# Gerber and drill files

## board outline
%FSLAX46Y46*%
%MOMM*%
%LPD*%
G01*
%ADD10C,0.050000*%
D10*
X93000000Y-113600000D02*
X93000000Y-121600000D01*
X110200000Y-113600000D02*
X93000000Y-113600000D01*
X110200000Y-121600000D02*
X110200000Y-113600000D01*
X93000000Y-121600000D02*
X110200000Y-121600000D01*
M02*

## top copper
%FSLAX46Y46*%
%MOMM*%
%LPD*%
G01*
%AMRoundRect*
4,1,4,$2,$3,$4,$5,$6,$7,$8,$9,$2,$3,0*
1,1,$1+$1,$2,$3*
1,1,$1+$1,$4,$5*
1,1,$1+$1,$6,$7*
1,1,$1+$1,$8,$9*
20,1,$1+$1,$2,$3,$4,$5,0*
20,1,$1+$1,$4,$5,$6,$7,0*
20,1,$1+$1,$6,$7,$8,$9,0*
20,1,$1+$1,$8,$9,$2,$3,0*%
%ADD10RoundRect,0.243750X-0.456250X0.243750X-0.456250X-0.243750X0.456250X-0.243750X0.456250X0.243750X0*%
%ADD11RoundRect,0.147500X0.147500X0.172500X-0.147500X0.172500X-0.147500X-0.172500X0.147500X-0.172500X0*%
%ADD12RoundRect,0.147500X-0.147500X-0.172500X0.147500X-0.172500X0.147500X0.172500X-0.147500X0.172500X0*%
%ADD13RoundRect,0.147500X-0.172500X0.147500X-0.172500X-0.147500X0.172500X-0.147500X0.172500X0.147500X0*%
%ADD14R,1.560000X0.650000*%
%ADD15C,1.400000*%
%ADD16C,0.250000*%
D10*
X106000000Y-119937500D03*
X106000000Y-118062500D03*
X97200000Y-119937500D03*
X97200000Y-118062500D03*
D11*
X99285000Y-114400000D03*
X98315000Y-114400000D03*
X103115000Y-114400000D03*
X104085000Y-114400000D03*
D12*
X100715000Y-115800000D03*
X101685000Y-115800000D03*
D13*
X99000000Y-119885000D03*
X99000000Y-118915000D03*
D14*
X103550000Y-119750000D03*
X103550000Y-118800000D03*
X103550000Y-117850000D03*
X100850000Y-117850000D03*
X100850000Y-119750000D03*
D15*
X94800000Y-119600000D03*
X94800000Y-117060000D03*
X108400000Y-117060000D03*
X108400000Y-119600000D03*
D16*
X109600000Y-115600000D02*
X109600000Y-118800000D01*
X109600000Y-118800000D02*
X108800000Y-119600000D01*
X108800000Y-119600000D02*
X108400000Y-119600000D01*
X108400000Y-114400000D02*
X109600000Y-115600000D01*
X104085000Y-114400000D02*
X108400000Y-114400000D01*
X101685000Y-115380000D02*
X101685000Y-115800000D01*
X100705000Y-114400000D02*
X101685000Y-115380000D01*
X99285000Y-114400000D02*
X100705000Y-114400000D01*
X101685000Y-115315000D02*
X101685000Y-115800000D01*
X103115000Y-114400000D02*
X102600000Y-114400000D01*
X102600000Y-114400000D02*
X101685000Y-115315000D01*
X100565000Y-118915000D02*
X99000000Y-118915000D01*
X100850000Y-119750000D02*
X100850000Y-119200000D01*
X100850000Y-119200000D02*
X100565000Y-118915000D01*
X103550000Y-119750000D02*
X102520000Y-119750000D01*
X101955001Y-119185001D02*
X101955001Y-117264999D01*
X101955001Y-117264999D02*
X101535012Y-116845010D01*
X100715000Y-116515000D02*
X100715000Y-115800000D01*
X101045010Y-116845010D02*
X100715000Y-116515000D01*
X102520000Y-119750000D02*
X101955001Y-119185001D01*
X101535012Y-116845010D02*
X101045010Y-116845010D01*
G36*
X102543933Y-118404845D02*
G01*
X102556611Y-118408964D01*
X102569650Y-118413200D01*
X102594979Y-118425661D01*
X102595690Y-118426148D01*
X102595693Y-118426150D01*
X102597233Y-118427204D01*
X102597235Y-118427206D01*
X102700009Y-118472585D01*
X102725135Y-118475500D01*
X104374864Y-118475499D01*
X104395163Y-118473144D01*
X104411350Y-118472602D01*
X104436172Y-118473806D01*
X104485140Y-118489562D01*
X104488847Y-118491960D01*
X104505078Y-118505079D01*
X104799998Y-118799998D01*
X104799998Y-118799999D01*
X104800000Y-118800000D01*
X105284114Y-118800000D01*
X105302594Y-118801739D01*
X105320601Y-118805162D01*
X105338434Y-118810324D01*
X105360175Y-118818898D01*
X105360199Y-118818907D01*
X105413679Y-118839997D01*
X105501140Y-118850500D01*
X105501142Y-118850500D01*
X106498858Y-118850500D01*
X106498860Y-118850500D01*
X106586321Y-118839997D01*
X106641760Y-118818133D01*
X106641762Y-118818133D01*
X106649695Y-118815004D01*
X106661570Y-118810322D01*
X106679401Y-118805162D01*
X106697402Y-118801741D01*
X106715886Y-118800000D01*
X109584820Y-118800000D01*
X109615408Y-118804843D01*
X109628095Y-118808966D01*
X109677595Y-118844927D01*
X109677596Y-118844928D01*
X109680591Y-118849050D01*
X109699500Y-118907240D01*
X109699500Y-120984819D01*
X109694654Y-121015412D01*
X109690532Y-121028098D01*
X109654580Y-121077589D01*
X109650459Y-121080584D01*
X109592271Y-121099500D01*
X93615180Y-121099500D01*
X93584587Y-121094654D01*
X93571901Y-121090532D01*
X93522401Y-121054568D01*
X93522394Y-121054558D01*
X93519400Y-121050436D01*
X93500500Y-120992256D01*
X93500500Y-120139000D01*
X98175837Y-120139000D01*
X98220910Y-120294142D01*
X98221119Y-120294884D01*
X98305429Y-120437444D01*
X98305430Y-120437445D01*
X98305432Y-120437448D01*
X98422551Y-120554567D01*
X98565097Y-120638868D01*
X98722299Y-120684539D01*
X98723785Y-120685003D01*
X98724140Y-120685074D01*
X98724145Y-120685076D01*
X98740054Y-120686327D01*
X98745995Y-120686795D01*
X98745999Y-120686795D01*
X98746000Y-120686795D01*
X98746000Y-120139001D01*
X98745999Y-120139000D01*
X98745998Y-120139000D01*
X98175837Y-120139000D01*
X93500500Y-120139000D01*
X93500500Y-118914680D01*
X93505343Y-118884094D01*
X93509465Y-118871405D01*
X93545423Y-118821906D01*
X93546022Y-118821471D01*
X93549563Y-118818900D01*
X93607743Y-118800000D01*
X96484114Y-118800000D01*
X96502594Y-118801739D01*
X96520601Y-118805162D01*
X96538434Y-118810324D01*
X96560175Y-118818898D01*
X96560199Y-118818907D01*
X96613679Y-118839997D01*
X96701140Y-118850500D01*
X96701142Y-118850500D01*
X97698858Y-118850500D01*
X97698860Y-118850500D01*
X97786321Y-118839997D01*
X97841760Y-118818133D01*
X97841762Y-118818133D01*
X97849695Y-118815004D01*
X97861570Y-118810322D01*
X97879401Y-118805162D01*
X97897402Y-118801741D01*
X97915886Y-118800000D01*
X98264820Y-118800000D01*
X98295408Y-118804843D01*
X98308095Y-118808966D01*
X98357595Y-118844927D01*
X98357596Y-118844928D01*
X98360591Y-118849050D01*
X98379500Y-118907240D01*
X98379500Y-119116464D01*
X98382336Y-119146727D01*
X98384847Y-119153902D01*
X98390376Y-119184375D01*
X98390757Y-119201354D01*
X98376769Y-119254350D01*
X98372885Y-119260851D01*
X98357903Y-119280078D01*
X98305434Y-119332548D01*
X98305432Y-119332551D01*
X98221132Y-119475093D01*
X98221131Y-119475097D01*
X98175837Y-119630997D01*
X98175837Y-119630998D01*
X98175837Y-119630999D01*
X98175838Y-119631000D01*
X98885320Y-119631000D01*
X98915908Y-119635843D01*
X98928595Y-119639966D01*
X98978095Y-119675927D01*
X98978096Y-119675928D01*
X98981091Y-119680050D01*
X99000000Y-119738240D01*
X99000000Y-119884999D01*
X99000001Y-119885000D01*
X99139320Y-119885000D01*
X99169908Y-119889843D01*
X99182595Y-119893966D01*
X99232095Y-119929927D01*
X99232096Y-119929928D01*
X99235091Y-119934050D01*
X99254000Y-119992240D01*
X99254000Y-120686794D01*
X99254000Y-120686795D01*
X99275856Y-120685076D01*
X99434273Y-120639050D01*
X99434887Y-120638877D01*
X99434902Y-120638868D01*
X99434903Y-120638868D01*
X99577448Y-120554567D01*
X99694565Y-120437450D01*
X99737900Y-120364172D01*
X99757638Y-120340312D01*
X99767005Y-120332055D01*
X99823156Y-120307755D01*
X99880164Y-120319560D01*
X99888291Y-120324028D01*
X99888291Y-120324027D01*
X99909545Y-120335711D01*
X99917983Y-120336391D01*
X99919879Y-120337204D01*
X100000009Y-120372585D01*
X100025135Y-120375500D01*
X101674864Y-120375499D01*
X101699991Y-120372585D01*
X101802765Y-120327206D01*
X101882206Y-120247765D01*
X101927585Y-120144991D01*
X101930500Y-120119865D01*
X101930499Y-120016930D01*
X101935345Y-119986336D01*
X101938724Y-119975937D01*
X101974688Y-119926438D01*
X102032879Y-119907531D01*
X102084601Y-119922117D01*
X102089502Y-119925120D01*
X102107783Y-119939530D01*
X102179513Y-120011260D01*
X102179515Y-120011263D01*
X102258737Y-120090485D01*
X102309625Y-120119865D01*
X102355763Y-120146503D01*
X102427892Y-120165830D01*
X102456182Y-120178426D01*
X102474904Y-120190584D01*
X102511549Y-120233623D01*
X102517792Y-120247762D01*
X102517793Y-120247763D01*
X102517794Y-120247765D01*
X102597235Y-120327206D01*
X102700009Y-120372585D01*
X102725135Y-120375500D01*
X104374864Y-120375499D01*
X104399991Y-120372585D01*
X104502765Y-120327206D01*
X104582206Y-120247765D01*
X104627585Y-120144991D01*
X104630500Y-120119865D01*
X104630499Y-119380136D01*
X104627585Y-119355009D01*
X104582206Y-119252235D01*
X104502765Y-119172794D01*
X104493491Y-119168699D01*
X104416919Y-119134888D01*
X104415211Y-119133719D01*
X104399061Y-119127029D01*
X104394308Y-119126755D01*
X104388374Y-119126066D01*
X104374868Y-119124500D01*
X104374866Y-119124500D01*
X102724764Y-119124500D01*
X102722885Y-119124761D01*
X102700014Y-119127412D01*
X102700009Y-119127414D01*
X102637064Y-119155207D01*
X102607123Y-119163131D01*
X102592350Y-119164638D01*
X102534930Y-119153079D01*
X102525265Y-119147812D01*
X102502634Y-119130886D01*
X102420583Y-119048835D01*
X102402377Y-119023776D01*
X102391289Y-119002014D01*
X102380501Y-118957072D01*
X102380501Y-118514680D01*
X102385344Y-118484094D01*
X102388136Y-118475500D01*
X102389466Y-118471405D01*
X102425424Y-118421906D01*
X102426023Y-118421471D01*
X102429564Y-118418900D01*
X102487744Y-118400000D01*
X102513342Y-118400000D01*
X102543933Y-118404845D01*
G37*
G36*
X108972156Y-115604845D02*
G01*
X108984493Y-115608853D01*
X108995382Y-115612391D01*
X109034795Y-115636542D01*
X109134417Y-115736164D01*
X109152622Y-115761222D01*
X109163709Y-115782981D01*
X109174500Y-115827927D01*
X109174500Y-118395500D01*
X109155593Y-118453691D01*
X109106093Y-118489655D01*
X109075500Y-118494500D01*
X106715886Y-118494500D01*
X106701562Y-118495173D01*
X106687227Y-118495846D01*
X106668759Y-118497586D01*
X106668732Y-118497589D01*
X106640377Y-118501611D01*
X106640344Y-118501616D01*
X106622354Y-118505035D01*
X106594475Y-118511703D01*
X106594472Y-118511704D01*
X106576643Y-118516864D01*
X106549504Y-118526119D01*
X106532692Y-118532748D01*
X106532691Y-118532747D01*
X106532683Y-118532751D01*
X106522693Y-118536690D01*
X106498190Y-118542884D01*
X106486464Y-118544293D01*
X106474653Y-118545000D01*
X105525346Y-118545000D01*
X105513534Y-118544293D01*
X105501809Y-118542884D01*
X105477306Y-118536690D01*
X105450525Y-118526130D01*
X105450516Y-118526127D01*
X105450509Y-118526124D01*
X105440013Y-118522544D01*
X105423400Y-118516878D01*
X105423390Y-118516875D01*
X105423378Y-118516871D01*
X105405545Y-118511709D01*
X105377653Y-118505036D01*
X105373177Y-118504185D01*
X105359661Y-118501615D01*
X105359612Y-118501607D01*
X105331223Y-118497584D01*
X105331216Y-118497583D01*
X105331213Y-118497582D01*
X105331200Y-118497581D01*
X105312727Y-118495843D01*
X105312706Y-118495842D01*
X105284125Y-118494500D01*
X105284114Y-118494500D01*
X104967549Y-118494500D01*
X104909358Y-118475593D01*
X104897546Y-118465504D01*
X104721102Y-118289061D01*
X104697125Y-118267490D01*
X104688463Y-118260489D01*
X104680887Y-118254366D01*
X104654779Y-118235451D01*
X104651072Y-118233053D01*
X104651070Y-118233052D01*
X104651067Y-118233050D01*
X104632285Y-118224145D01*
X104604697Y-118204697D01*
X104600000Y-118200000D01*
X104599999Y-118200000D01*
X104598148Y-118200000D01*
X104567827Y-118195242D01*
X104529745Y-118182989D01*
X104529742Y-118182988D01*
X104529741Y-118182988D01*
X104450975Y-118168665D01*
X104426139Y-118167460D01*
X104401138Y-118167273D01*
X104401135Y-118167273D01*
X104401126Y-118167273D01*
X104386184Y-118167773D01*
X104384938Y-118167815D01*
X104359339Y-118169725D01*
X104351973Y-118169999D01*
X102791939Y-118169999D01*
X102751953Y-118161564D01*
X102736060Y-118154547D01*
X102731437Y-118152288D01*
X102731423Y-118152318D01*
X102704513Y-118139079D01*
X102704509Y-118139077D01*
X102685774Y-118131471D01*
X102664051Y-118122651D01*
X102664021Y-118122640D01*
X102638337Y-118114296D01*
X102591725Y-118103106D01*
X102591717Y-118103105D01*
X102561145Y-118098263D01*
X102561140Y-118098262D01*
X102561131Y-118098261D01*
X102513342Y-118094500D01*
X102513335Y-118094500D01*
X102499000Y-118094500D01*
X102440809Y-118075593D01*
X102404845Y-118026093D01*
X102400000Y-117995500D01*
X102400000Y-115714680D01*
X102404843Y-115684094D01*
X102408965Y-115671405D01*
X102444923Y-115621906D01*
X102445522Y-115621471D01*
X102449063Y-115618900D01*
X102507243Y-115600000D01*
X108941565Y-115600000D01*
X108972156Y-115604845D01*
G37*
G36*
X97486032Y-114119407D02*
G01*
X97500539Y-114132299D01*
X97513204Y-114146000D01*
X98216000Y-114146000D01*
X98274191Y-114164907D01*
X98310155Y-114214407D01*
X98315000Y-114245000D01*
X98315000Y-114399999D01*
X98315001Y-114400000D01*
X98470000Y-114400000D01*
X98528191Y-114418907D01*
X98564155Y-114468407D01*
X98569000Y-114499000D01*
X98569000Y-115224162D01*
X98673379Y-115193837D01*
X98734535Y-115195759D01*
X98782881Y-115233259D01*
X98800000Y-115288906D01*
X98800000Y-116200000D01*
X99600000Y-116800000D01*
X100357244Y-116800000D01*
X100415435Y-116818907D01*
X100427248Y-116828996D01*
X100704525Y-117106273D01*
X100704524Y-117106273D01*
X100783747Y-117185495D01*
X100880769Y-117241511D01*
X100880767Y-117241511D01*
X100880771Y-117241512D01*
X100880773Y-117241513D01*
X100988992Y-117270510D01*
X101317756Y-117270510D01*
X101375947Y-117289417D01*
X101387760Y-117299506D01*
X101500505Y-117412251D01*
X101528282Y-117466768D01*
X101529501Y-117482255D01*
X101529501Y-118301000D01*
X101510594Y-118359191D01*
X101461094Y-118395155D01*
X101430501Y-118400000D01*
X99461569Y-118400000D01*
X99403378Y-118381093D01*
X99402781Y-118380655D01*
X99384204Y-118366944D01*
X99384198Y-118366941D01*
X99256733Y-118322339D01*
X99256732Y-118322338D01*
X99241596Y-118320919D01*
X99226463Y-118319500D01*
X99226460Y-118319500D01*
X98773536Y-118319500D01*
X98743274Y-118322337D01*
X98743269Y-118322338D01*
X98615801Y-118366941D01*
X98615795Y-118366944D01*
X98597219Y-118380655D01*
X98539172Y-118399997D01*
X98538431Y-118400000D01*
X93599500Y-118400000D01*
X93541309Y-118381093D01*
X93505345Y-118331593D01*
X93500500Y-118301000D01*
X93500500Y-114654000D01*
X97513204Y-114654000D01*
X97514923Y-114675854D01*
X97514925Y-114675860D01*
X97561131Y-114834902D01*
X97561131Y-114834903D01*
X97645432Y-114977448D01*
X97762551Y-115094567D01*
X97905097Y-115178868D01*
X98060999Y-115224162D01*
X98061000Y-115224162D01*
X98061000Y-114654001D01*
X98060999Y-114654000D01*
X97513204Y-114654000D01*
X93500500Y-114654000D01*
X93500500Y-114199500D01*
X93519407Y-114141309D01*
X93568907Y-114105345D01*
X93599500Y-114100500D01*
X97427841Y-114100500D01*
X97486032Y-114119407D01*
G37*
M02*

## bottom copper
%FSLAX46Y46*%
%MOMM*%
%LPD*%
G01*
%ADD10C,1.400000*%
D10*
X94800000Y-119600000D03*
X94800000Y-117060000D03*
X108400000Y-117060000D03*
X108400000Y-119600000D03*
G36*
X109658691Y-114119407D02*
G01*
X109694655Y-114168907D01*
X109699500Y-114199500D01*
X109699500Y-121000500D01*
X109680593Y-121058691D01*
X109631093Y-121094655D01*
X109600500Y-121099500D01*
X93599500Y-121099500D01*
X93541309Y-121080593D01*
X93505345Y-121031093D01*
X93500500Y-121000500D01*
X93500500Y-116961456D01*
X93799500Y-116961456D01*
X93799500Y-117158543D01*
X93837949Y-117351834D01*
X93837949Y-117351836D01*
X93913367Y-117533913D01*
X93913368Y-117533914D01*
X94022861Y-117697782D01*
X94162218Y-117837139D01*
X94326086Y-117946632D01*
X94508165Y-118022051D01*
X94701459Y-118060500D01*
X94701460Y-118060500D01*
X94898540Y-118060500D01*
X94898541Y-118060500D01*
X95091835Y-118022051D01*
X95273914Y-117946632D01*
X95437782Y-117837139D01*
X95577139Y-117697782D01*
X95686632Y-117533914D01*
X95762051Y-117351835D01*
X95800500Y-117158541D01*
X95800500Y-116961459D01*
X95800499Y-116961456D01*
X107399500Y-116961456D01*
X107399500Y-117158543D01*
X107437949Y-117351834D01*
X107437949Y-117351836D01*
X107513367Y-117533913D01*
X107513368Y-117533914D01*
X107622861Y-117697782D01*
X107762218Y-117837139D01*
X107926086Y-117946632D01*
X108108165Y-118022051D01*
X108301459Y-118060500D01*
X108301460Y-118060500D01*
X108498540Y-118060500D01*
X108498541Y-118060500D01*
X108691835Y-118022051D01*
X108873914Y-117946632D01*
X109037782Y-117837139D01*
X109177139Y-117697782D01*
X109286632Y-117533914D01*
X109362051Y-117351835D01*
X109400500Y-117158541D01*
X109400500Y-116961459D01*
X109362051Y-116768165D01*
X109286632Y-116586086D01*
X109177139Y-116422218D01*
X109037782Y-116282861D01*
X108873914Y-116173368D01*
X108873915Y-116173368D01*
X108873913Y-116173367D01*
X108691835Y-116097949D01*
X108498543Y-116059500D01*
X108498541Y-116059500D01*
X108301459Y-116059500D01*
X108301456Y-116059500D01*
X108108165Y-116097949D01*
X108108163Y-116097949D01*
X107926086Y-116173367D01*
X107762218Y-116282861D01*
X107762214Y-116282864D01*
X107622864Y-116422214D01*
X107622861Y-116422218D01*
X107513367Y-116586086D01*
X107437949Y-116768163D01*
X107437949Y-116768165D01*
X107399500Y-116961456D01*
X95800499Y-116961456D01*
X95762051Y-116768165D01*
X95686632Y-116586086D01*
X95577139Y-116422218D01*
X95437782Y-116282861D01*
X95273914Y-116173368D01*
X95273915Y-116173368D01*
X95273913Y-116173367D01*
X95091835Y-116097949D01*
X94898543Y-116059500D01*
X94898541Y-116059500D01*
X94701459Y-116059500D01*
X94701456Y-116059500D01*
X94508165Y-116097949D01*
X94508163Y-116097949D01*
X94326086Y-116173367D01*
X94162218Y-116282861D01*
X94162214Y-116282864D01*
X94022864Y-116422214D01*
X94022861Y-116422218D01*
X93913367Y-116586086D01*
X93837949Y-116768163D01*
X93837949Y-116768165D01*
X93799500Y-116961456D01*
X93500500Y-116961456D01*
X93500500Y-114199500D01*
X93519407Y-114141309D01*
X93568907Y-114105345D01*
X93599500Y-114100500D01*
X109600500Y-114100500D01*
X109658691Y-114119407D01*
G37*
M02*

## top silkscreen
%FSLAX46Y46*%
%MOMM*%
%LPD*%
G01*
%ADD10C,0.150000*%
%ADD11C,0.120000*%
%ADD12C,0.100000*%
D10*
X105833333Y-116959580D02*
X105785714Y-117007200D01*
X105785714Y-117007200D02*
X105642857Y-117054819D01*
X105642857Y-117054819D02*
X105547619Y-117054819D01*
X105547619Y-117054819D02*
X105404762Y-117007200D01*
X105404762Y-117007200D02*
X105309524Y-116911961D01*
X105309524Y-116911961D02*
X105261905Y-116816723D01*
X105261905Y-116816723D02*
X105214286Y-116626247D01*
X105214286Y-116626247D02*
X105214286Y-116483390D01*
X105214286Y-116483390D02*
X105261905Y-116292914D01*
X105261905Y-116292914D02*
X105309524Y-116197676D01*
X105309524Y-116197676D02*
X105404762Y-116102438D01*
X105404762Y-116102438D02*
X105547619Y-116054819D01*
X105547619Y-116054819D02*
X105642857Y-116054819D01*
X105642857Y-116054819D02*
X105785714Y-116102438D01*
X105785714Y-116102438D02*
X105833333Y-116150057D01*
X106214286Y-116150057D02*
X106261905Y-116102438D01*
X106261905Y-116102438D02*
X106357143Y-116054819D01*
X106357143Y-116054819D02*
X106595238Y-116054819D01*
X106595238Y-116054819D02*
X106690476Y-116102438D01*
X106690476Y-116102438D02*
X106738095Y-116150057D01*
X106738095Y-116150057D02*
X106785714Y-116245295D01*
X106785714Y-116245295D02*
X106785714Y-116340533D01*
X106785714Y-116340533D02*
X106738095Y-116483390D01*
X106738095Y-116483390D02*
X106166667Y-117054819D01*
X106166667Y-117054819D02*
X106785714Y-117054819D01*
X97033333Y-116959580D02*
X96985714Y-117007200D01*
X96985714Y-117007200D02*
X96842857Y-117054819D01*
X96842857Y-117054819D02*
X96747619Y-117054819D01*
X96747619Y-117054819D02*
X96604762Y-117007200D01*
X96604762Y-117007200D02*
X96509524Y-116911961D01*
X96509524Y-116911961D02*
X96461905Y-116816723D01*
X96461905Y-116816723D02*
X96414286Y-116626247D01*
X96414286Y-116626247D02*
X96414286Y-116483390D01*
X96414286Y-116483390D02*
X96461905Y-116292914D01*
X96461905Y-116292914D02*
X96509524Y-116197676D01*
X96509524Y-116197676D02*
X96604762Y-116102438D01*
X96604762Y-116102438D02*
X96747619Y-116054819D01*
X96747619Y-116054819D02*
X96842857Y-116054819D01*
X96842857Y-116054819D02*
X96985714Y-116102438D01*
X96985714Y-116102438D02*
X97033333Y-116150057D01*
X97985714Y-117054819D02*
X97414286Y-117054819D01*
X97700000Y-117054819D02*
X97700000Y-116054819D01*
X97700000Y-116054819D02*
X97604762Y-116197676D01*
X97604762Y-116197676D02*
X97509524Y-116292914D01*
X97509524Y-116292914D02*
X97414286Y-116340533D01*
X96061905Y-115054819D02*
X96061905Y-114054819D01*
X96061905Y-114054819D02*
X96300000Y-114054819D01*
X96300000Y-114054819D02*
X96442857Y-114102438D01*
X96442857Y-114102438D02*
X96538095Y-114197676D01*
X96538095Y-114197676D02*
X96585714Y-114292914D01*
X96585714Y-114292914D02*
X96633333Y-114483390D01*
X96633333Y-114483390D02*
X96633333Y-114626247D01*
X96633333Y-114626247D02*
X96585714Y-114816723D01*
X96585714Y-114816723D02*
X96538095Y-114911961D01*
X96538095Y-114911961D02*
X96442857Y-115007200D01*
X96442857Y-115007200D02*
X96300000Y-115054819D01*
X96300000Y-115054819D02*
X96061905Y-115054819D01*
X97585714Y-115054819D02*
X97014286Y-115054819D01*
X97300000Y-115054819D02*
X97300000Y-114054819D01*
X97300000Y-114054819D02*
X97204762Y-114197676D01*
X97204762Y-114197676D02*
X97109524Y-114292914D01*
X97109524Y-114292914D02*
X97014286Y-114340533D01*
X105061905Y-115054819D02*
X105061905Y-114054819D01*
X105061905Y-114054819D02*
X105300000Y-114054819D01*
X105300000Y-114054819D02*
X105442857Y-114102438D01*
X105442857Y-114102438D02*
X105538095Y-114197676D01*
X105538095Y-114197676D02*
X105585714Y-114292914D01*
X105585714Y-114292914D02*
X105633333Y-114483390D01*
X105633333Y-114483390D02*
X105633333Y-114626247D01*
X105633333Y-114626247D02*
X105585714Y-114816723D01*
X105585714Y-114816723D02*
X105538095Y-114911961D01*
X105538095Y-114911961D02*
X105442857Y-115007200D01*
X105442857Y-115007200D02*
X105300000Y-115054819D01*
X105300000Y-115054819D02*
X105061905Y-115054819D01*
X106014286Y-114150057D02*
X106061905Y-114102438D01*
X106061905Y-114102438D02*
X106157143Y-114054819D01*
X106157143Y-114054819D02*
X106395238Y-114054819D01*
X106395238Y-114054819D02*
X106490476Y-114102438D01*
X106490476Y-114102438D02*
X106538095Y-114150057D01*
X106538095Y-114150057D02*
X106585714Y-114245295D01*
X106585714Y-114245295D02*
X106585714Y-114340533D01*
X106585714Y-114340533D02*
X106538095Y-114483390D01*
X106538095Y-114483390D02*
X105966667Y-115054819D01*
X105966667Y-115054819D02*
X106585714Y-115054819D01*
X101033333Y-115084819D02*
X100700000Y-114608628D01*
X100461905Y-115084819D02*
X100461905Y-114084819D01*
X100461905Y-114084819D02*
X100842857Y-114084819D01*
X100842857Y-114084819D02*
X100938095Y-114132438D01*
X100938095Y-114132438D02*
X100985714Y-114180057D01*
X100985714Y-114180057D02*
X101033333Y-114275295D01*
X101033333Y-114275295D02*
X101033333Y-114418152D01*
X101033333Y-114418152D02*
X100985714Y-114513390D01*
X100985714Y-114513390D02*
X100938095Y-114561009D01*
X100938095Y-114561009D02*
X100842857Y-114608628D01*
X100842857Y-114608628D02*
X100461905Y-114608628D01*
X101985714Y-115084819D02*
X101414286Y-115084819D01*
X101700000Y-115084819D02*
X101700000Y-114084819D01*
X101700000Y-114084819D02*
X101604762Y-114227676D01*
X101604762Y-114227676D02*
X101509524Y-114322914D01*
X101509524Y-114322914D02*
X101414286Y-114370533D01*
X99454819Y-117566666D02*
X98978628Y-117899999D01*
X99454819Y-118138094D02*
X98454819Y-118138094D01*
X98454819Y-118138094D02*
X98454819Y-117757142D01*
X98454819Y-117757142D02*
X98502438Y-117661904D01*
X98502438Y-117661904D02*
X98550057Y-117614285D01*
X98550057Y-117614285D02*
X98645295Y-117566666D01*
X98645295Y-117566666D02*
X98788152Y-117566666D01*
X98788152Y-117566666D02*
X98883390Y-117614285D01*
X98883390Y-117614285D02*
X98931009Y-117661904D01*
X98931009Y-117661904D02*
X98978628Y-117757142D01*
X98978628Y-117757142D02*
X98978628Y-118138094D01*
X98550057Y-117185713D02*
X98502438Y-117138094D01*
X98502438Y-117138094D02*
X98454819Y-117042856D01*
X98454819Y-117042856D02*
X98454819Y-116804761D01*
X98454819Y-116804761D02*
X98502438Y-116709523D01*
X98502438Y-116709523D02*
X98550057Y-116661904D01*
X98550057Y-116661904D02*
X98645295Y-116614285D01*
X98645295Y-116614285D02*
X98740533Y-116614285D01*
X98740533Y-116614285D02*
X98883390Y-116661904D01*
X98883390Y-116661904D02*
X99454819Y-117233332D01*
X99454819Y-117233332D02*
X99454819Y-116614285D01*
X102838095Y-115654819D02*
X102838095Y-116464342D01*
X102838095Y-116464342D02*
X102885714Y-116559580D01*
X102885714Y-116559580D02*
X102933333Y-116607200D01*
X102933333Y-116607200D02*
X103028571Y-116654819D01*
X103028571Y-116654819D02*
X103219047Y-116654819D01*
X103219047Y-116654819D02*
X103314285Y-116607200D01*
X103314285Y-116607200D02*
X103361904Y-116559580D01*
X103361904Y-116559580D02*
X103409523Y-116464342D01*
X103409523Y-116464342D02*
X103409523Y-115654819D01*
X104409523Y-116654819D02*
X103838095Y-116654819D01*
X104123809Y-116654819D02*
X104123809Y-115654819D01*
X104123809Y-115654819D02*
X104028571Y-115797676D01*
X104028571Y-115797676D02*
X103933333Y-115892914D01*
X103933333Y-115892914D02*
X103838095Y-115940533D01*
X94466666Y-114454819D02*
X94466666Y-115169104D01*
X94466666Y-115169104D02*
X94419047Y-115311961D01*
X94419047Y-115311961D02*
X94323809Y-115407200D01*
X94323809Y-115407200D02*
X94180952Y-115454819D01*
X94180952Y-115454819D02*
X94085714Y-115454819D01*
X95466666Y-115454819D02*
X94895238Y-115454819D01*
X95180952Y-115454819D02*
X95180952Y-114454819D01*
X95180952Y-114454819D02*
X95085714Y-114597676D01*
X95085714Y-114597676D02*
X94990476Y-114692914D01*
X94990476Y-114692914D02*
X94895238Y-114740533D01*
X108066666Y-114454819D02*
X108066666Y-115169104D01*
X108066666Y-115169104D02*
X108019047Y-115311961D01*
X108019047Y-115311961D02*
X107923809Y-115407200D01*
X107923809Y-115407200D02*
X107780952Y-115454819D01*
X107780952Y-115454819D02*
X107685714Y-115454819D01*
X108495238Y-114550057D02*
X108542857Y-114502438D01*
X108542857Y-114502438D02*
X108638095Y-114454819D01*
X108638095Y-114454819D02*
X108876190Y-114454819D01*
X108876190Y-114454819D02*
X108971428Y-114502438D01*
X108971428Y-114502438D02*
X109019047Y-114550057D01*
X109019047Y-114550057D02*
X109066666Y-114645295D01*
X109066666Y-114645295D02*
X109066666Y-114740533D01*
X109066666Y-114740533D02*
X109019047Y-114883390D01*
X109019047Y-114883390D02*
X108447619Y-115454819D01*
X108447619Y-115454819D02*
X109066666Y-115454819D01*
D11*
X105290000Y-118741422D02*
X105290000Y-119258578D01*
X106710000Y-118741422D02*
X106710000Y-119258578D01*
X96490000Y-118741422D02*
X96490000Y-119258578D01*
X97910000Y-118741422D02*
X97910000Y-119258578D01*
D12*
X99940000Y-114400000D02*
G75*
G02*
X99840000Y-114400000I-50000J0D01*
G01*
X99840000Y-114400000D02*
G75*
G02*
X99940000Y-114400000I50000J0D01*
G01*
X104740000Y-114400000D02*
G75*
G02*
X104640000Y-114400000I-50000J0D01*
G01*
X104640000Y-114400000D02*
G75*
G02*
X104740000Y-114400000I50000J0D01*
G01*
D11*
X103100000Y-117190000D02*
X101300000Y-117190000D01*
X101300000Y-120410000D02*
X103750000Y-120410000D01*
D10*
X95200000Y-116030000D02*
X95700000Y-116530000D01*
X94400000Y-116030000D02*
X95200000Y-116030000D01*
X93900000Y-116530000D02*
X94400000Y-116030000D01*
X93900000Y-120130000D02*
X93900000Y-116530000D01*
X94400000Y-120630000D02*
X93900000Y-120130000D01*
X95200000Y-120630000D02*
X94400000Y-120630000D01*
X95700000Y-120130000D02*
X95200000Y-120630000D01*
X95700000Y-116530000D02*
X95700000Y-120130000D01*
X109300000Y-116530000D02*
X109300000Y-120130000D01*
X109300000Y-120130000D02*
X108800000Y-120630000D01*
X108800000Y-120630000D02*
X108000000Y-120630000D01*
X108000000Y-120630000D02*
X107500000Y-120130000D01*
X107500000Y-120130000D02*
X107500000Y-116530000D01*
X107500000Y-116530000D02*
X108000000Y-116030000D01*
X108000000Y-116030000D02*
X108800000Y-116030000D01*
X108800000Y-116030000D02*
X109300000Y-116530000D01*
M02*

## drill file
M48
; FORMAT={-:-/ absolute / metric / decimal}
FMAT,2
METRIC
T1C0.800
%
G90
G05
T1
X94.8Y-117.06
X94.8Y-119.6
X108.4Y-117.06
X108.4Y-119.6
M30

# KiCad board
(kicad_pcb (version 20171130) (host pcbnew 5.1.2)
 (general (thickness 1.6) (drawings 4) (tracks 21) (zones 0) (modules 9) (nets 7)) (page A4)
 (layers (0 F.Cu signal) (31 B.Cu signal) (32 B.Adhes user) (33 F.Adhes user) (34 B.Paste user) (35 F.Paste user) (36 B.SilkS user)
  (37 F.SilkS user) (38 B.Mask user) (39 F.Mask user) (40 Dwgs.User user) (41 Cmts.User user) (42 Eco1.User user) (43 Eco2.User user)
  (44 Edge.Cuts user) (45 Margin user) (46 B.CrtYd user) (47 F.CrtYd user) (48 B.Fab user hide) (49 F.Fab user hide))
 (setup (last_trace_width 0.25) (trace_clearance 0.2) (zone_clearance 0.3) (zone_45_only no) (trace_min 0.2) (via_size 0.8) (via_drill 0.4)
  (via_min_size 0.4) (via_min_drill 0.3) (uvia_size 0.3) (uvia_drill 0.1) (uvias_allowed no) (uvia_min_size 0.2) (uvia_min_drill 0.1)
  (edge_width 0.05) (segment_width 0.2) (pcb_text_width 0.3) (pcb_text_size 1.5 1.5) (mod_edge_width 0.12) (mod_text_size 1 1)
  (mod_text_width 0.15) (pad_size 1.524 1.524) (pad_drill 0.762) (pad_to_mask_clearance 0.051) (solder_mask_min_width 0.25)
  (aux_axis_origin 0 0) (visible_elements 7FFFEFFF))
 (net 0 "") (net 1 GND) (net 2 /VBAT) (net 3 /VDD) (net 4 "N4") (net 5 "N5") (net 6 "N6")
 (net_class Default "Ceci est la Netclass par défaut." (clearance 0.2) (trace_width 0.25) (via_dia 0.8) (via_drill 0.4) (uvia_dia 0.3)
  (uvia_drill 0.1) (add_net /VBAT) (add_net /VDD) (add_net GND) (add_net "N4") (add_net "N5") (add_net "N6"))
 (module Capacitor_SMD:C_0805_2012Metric (layer F.Cu) (at 106 119 270)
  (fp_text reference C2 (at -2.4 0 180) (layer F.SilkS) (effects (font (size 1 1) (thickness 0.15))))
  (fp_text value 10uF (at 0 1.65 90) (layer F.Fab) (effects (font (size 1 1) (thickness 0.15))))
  (fp_line (start -0.258578 0.71) (end 0.258578 0.71) (layer F.SilkS) (width 0.12))
  (fp_line (start -0.258578 -0.71) (end 0.258578 -0.71) (layer F.SilkS) (width 0.12))
  (pad 2 smd roundrect (at 0.9375 0 270) (size 0.975 1.4) (layers F.Cu F.Paste F.Mask) (roundrect_rratio 0.25) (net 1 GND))
  (pad 1 smd roundrect (at -0.9375 0 270) (size 0.975 1.4) (layers F.Cu F.Paste F.Mask) (roundrect_rratio 0.25) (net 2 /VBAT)))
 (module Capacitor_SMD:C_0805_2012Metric (layer F.Cu) (at 97.2 119 270)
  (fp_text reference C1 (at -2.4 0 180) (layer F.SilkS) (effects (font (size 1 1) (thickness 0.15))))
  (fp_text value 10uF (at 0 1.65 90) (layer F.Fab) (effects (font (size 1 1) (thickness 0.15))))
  (fp_line (start -0.258578 0.71) (end 0.258578 0.71) (layer F.SilkS) (width 0.12))
  (fp_line (start -0.258578 -0.71) (end 0.258578 -0.71) (layer F.SilkS) (width 0.12))
  (pad 2 smd roundrect (at 0.9375 0 270) (size 0.975 1.4) (layers F.Cu F.Paste F.Mask) (roundrect_rratio 0.25) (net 1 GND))
  (pad 1 smd roundrect (at -0.9375 0 270) (size 0.975 1.4) (layers F.Cu F.Paste F.Mask) (roundrect_rratio 0.25) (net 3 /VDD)))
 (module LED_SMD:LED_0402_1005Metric (layer F.Cu) (at 98.8 114.4 180) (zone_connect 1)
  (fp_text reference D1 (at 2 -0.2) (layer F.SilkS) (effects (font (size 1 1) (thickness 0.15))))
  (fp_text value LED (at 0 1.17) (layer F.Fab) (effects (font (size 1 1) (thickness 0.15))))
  (fp_circle (center -1.09 0) (end -1.04 0) (layer F.SilkS) (width 0.1))
  (pad 1 smd roundrect (at -0.485 0 180) (size 0.59 0.64) (layers F.Cu F.Paste F.Mask) (roundrect_rratio 0.25) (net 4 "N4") (zone_connect 1))
  (pad 2 smd roundrect (at 0.485 0 180) (size 0.59 0.64) (layers F.Cu F.Paste F.Mask) (roundrect_rratio 0.25) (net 3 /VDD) (zone_connect 1)))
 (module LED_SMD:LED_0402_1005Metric (layer F.Cu) (at 103.6 114.4 180)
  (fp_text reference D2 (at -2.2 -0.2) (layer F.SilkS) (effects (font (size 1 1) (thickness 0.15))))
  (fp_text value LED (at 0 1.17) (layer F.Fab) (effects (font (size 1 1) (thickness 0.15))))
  (fp_circle (center -1.09 0) (end -1.04 0) (layer F.SilkS) (width 0.1))
  (pad 2 smd roundrect (at 0.485 0 180) (size 0.59 0.64) (layers F.Cu F.Paste F.Mask) (roundrect_rratio 0.25) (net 4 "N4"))
  (pad 1 smd roundrect (at -0.485 0 180) (size 0.59 0.64) (layers F.Cu F.Paste F.Mask) (roundrect_rratio 0.25) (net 1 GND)))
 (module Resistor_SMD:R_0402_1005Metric (layer F.Cu) (at 101.2 115.8)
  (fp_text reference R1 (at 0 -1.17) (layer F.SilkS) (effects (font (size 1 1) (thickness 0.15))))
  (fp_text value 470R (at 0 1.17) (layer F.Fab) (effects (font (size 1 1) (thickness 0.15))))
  (pad 1 smd roundrect (at -0.485 0) (size 0.59 0.64) (layers F.Cu F.Paste F.Mask) (roundrect_rratio 0.25) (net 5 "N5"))
  (pad 2 smd roundrect (at 0.485 0) (size 0.59 0.64) (layers F.Cu F.Paste F.Mask) (roundrect_rratio 0.25) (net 4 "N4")))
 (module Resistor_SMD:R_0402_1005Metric (layer F.Cu) (at 99 119.4 270) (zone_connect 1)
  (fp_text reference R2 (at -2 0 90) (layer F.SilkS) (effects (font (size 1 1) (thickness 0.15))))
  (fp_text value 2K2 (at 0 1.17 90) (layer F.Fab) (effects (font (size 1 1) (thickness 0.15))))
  (pad 2 smd roundrect (at 0.485 0 270) (size 0.59 0.64) (layers F.Cu F.Paste F.Mask) (roundrect_rratio 0.25) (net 1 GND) (zone_connect 1))
  (pad 1 smd roundrect (at -0.485 0 270) (size 0.59 0.64) (layers F.Cu F.Paste F.Mask) (roundrect_rratio 0.25) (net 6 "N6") (zone_connect 1)))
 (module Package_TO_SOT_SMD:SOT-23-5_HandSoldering (layer F.Cu) (at 102.2 118.8 180)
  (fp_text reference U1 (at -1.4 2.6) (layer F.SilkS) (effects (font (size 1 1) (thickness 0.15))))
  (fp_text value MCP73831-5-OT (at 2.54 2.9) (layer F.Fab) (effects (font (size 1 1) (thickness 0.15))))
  (fp_line (start -0.9 1.61) (end 0.9 1.61) (layer F.SilkS) (width 0.12))
  (fp_line (start 0.9 -1.61) (end -1.55 -1.61) (layer F.SilkS) (width 0.12))
  (pad 1 smd rect (at -1.35 -0.95 180) (size 1.56 0.65) (layers F.Cu F.Paste F.Mask) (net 5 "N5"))
  (pad 2 smd rect (at -1.35 0 180) (size 1.56 0.65) (layers F.Cu F.Paste F.Mask) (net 1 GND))
  (pad 3 smd rect (at -1.35 0.95 180) (size 1.56 0.65) (layers F.Cu F.Paste F.Mask) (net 2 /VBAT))
  (pad 4 smd rect (at 1.35 0.95 180) (size 1.56 0.65) (layers F.Cu F.Paste F.Mask) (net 3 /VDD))
  (pad 5 smd rect (at 1.35 -0.95 180) (size 1.56 0.65) (layers F.Cu F.Paste F.Mask) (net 6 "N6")))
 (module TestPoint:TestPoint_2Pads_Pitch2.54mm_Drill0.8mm (layer F.Cu) (at 94.8 117.06 270)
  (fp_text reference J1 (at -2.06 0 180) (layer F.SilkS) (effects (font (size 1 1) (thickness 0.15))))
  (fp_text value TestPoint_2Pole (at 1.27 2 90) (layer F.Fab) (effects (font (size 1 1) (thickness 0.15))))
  (fp_line (start -1.03 -0.4) (end -0.53 -0.9) (layer F.SilkS) (width 0.15))
  (fp_line (start -1.03 0.4) (end -1.03 -0.4) (layer F.SilkS) (width 0.15))
  (fp_line (start -0.53 0.9) (end -1.03 0.4) (layer F.SilkS) (width 0.15))
  (fp_line (start 3.07 0.9) (end -0.53 0.9) (layer F.SilkS) (width 0.15))
  (fp_line (start 3.57 0.4) (end 3.07 0.9) (layer F.SilkS) (width 0.15))
  (fp_line (start 3.57 -0.4) (end 3.57 0.4) (layer F.SilkS) (width 0.15))
  (fp_line (start 3.07 -0.9) (end 3.57 -0.4) (layer F.SilkS) (width 0.15))
  (fp_line (start -0.53 -0.9) (end 3.07 -0.9) (layer F.SilkS) (width 0.15))
  (pad 2 thru_hole circle (at 2.54 0 270) (size 1.4 1.4) (drill 0.8) (layers *.Cu *.Mask) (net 1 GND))
  (pad 1 thru_hole circle (at 0 0 270) (size 1.4 1.4) (drill 0.8) (layers *.Cu *.Mask) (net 3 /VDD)))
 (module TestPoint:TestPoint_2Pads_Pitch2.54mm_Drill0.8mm (layer F.Cu) (at 108.4 117.06 270)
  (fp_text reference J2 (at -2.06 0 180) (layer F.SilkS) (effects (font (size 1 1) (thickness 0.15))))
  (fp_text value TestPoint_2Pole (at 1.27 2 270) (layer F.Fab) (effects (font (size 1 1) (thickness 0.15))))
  (fp_line (start -0.53 -0.9) (end 3.07 -0.9) (layer F.SilkS) (width 0.15))
  (fp_line (start 3.07 -0.9) (end 3.57 -0.4) (layer F.SilkS) (width 0.15))
  (fp_line (start 3.57 -0.4) (end 3.57 0.4) (layer F.SilkS) (width 0.15))
  (fp_line (start 3.57 0.4) (end 3.07 0.9) (layer F.SilkS) (width 0.15))
  (fp_line (start 3.07 0.9) (end -0.53 0.9) (layer F.SilkS) (width 0.15))
  (fp_line (start -0.53 0.9) (end -1.03 0.4) (layer F.SilkS) (width 0.15))
  (fp_line (start -1.03 0.4) (end -1.03 -0.4) (layer F.SilkS) (width 0.15))
  (fp_line (start -1.03 -0.4) (end -0.53 -0.9) (layer F.SilkS) (width 0.15))
  (pad 1 thru_hole circle (at 0 0 270) (size 1.4 1.4) (drill 0.8) (layers *.Cu *.Mask) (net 2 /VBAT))
  (pad 2 thru_hole circle (at 2.54 0 270) (size 1.4 1.4) (drill 0.8) (layers *.Cu *.Mask) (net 1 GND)))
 (gr_line (start 93 113.6) (end 93 121.6) (layer Edge.Cuts) (width 0.05))
 (gr_line (start 110.2 113.6) (end 93 113.6) (layer Edge.Cuts) (width 0.05))
 (gr_line (start 110.2 121.6) (end 110.2 113.6) (layer Edge.Cuts) (width 0.05))
 (gr_line (start 93 121.6) (end 110.2 121.6) (layer Edge.Cuts) (width 0.05))
 (segment (start 109.6 115.6) (end 109.6 118.8) (width 0.25) (layer F.Cu) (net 1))
 (segment (start 109.6 118.8) (end 108.8 119.6) (width 0.25) (layer F.Cu) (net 1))
 (segment (start 108.8 119.6) (end 108.4 119.6) (width 0.25) (layer F.Cu) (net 1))
 (segment (start 108.4 114.4) (end 109.6 115.6) (width 0.25) (layer F.Cu) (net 1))
 (segment (start 104.085 114.4) (end 108.4 114.4) (width 0.25) (layer F.Cu) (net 1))
 (segment (start 101.685 115.38) (end 101.685 115.8) (width 0.25) (layer F.Cu) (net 4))
 (segment (start 100.705 114.4) (end 101.685 115.38) (width 0.25) (layer F.Cu) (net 4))
 (segment (start 99.285 114.4) (end 100.705 114.4) (width 0.25) (layer F.Cu) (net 4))
 (segment (start 101.685 115.315) (end 101.685 115.8) (width 0.25) (layer F.Cu) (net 4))
 (segment (start 103.115 114.4) (end 102.6 114.4) (width 0.25) (layer F.Cu) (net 4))
 (segment (start 102.6 114.4) (end 101.685 115.315) (width 0.25) (layer F.Cu) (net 4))
 (segment (start 100.565 118.915) (end 99 118.915) (width 0.25) (layer F.Cu) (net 6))
 (segment (start 100.85 119.75) (end 100.85 119.2) (width 0.25) (layer F.Cu) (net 6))
 (segment (start 100.85 119.2) (end 100.565 118.915) (width 0.25) (layer F.Cu) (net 6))
 (segment (start 103.55 119.75) (end 102.52 119.75) (width 0.25) (layer F.Cu) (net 5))
 (segment (start 101.955001 119.185001) (end 101.955001 117.264999) (width 0.25) (layer F.Cu) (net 5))
 (segment (start 101.955001 117.264999) (end 101.535012 116.84501) (width 0.25) (layer F.Cu) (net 5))
 (segment (start 100.715 116.515) (end 100.715 115.8) (width 0.25) (layer F.Cu) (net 5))
 (segment (start 101.04501 116.84501) (end 100.715 116.515) (width 0.25) (layer F.Cu) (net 5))
 (segment (start 102.52 119.75) (end 101.955001 119.185001) (width 0.25) (layer F.Cu) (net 5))
 (segment (start 101.535012 116.84501) (end 101.04501 116.84501) (width 0.25) (layer F.Cu) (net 5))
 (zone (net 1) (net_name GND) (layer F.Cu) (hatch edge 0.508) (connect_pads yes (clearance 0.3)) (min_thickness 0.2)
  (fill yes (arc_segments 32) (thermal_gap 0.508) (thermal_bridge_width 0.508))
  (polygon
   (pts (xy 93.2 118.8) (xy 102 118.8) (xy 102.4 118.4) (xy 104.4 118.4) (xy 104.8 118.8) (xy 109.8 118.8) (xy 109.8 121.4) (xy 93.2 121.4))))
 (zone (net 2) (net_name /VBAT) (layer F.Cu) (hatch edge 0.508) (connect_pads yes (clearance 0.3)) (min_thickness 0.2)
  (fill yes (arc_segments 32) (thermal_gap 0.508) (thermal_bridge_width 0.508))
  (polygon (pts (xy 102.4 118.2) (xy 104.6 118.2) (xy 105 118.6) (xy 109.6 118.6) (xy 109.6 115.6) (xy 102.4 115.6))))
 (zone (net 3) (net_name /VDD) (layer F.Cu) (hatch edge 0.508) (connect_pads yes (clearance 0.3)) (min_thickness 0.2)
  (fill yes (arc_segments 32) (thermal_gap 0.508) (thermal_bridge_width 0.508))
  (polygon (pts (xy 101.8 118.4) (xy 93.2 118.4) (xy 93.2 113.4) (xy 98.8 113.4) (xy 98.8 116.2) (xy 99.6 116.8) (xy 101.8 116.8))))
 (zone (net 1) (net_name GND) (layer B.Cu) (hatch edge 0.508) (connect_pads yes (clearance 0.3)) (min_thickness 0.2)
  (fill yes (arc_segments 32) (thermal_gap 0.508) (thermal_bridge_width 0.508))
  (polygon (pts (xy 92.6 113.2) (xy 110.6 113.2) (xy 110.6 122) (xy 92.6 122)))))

